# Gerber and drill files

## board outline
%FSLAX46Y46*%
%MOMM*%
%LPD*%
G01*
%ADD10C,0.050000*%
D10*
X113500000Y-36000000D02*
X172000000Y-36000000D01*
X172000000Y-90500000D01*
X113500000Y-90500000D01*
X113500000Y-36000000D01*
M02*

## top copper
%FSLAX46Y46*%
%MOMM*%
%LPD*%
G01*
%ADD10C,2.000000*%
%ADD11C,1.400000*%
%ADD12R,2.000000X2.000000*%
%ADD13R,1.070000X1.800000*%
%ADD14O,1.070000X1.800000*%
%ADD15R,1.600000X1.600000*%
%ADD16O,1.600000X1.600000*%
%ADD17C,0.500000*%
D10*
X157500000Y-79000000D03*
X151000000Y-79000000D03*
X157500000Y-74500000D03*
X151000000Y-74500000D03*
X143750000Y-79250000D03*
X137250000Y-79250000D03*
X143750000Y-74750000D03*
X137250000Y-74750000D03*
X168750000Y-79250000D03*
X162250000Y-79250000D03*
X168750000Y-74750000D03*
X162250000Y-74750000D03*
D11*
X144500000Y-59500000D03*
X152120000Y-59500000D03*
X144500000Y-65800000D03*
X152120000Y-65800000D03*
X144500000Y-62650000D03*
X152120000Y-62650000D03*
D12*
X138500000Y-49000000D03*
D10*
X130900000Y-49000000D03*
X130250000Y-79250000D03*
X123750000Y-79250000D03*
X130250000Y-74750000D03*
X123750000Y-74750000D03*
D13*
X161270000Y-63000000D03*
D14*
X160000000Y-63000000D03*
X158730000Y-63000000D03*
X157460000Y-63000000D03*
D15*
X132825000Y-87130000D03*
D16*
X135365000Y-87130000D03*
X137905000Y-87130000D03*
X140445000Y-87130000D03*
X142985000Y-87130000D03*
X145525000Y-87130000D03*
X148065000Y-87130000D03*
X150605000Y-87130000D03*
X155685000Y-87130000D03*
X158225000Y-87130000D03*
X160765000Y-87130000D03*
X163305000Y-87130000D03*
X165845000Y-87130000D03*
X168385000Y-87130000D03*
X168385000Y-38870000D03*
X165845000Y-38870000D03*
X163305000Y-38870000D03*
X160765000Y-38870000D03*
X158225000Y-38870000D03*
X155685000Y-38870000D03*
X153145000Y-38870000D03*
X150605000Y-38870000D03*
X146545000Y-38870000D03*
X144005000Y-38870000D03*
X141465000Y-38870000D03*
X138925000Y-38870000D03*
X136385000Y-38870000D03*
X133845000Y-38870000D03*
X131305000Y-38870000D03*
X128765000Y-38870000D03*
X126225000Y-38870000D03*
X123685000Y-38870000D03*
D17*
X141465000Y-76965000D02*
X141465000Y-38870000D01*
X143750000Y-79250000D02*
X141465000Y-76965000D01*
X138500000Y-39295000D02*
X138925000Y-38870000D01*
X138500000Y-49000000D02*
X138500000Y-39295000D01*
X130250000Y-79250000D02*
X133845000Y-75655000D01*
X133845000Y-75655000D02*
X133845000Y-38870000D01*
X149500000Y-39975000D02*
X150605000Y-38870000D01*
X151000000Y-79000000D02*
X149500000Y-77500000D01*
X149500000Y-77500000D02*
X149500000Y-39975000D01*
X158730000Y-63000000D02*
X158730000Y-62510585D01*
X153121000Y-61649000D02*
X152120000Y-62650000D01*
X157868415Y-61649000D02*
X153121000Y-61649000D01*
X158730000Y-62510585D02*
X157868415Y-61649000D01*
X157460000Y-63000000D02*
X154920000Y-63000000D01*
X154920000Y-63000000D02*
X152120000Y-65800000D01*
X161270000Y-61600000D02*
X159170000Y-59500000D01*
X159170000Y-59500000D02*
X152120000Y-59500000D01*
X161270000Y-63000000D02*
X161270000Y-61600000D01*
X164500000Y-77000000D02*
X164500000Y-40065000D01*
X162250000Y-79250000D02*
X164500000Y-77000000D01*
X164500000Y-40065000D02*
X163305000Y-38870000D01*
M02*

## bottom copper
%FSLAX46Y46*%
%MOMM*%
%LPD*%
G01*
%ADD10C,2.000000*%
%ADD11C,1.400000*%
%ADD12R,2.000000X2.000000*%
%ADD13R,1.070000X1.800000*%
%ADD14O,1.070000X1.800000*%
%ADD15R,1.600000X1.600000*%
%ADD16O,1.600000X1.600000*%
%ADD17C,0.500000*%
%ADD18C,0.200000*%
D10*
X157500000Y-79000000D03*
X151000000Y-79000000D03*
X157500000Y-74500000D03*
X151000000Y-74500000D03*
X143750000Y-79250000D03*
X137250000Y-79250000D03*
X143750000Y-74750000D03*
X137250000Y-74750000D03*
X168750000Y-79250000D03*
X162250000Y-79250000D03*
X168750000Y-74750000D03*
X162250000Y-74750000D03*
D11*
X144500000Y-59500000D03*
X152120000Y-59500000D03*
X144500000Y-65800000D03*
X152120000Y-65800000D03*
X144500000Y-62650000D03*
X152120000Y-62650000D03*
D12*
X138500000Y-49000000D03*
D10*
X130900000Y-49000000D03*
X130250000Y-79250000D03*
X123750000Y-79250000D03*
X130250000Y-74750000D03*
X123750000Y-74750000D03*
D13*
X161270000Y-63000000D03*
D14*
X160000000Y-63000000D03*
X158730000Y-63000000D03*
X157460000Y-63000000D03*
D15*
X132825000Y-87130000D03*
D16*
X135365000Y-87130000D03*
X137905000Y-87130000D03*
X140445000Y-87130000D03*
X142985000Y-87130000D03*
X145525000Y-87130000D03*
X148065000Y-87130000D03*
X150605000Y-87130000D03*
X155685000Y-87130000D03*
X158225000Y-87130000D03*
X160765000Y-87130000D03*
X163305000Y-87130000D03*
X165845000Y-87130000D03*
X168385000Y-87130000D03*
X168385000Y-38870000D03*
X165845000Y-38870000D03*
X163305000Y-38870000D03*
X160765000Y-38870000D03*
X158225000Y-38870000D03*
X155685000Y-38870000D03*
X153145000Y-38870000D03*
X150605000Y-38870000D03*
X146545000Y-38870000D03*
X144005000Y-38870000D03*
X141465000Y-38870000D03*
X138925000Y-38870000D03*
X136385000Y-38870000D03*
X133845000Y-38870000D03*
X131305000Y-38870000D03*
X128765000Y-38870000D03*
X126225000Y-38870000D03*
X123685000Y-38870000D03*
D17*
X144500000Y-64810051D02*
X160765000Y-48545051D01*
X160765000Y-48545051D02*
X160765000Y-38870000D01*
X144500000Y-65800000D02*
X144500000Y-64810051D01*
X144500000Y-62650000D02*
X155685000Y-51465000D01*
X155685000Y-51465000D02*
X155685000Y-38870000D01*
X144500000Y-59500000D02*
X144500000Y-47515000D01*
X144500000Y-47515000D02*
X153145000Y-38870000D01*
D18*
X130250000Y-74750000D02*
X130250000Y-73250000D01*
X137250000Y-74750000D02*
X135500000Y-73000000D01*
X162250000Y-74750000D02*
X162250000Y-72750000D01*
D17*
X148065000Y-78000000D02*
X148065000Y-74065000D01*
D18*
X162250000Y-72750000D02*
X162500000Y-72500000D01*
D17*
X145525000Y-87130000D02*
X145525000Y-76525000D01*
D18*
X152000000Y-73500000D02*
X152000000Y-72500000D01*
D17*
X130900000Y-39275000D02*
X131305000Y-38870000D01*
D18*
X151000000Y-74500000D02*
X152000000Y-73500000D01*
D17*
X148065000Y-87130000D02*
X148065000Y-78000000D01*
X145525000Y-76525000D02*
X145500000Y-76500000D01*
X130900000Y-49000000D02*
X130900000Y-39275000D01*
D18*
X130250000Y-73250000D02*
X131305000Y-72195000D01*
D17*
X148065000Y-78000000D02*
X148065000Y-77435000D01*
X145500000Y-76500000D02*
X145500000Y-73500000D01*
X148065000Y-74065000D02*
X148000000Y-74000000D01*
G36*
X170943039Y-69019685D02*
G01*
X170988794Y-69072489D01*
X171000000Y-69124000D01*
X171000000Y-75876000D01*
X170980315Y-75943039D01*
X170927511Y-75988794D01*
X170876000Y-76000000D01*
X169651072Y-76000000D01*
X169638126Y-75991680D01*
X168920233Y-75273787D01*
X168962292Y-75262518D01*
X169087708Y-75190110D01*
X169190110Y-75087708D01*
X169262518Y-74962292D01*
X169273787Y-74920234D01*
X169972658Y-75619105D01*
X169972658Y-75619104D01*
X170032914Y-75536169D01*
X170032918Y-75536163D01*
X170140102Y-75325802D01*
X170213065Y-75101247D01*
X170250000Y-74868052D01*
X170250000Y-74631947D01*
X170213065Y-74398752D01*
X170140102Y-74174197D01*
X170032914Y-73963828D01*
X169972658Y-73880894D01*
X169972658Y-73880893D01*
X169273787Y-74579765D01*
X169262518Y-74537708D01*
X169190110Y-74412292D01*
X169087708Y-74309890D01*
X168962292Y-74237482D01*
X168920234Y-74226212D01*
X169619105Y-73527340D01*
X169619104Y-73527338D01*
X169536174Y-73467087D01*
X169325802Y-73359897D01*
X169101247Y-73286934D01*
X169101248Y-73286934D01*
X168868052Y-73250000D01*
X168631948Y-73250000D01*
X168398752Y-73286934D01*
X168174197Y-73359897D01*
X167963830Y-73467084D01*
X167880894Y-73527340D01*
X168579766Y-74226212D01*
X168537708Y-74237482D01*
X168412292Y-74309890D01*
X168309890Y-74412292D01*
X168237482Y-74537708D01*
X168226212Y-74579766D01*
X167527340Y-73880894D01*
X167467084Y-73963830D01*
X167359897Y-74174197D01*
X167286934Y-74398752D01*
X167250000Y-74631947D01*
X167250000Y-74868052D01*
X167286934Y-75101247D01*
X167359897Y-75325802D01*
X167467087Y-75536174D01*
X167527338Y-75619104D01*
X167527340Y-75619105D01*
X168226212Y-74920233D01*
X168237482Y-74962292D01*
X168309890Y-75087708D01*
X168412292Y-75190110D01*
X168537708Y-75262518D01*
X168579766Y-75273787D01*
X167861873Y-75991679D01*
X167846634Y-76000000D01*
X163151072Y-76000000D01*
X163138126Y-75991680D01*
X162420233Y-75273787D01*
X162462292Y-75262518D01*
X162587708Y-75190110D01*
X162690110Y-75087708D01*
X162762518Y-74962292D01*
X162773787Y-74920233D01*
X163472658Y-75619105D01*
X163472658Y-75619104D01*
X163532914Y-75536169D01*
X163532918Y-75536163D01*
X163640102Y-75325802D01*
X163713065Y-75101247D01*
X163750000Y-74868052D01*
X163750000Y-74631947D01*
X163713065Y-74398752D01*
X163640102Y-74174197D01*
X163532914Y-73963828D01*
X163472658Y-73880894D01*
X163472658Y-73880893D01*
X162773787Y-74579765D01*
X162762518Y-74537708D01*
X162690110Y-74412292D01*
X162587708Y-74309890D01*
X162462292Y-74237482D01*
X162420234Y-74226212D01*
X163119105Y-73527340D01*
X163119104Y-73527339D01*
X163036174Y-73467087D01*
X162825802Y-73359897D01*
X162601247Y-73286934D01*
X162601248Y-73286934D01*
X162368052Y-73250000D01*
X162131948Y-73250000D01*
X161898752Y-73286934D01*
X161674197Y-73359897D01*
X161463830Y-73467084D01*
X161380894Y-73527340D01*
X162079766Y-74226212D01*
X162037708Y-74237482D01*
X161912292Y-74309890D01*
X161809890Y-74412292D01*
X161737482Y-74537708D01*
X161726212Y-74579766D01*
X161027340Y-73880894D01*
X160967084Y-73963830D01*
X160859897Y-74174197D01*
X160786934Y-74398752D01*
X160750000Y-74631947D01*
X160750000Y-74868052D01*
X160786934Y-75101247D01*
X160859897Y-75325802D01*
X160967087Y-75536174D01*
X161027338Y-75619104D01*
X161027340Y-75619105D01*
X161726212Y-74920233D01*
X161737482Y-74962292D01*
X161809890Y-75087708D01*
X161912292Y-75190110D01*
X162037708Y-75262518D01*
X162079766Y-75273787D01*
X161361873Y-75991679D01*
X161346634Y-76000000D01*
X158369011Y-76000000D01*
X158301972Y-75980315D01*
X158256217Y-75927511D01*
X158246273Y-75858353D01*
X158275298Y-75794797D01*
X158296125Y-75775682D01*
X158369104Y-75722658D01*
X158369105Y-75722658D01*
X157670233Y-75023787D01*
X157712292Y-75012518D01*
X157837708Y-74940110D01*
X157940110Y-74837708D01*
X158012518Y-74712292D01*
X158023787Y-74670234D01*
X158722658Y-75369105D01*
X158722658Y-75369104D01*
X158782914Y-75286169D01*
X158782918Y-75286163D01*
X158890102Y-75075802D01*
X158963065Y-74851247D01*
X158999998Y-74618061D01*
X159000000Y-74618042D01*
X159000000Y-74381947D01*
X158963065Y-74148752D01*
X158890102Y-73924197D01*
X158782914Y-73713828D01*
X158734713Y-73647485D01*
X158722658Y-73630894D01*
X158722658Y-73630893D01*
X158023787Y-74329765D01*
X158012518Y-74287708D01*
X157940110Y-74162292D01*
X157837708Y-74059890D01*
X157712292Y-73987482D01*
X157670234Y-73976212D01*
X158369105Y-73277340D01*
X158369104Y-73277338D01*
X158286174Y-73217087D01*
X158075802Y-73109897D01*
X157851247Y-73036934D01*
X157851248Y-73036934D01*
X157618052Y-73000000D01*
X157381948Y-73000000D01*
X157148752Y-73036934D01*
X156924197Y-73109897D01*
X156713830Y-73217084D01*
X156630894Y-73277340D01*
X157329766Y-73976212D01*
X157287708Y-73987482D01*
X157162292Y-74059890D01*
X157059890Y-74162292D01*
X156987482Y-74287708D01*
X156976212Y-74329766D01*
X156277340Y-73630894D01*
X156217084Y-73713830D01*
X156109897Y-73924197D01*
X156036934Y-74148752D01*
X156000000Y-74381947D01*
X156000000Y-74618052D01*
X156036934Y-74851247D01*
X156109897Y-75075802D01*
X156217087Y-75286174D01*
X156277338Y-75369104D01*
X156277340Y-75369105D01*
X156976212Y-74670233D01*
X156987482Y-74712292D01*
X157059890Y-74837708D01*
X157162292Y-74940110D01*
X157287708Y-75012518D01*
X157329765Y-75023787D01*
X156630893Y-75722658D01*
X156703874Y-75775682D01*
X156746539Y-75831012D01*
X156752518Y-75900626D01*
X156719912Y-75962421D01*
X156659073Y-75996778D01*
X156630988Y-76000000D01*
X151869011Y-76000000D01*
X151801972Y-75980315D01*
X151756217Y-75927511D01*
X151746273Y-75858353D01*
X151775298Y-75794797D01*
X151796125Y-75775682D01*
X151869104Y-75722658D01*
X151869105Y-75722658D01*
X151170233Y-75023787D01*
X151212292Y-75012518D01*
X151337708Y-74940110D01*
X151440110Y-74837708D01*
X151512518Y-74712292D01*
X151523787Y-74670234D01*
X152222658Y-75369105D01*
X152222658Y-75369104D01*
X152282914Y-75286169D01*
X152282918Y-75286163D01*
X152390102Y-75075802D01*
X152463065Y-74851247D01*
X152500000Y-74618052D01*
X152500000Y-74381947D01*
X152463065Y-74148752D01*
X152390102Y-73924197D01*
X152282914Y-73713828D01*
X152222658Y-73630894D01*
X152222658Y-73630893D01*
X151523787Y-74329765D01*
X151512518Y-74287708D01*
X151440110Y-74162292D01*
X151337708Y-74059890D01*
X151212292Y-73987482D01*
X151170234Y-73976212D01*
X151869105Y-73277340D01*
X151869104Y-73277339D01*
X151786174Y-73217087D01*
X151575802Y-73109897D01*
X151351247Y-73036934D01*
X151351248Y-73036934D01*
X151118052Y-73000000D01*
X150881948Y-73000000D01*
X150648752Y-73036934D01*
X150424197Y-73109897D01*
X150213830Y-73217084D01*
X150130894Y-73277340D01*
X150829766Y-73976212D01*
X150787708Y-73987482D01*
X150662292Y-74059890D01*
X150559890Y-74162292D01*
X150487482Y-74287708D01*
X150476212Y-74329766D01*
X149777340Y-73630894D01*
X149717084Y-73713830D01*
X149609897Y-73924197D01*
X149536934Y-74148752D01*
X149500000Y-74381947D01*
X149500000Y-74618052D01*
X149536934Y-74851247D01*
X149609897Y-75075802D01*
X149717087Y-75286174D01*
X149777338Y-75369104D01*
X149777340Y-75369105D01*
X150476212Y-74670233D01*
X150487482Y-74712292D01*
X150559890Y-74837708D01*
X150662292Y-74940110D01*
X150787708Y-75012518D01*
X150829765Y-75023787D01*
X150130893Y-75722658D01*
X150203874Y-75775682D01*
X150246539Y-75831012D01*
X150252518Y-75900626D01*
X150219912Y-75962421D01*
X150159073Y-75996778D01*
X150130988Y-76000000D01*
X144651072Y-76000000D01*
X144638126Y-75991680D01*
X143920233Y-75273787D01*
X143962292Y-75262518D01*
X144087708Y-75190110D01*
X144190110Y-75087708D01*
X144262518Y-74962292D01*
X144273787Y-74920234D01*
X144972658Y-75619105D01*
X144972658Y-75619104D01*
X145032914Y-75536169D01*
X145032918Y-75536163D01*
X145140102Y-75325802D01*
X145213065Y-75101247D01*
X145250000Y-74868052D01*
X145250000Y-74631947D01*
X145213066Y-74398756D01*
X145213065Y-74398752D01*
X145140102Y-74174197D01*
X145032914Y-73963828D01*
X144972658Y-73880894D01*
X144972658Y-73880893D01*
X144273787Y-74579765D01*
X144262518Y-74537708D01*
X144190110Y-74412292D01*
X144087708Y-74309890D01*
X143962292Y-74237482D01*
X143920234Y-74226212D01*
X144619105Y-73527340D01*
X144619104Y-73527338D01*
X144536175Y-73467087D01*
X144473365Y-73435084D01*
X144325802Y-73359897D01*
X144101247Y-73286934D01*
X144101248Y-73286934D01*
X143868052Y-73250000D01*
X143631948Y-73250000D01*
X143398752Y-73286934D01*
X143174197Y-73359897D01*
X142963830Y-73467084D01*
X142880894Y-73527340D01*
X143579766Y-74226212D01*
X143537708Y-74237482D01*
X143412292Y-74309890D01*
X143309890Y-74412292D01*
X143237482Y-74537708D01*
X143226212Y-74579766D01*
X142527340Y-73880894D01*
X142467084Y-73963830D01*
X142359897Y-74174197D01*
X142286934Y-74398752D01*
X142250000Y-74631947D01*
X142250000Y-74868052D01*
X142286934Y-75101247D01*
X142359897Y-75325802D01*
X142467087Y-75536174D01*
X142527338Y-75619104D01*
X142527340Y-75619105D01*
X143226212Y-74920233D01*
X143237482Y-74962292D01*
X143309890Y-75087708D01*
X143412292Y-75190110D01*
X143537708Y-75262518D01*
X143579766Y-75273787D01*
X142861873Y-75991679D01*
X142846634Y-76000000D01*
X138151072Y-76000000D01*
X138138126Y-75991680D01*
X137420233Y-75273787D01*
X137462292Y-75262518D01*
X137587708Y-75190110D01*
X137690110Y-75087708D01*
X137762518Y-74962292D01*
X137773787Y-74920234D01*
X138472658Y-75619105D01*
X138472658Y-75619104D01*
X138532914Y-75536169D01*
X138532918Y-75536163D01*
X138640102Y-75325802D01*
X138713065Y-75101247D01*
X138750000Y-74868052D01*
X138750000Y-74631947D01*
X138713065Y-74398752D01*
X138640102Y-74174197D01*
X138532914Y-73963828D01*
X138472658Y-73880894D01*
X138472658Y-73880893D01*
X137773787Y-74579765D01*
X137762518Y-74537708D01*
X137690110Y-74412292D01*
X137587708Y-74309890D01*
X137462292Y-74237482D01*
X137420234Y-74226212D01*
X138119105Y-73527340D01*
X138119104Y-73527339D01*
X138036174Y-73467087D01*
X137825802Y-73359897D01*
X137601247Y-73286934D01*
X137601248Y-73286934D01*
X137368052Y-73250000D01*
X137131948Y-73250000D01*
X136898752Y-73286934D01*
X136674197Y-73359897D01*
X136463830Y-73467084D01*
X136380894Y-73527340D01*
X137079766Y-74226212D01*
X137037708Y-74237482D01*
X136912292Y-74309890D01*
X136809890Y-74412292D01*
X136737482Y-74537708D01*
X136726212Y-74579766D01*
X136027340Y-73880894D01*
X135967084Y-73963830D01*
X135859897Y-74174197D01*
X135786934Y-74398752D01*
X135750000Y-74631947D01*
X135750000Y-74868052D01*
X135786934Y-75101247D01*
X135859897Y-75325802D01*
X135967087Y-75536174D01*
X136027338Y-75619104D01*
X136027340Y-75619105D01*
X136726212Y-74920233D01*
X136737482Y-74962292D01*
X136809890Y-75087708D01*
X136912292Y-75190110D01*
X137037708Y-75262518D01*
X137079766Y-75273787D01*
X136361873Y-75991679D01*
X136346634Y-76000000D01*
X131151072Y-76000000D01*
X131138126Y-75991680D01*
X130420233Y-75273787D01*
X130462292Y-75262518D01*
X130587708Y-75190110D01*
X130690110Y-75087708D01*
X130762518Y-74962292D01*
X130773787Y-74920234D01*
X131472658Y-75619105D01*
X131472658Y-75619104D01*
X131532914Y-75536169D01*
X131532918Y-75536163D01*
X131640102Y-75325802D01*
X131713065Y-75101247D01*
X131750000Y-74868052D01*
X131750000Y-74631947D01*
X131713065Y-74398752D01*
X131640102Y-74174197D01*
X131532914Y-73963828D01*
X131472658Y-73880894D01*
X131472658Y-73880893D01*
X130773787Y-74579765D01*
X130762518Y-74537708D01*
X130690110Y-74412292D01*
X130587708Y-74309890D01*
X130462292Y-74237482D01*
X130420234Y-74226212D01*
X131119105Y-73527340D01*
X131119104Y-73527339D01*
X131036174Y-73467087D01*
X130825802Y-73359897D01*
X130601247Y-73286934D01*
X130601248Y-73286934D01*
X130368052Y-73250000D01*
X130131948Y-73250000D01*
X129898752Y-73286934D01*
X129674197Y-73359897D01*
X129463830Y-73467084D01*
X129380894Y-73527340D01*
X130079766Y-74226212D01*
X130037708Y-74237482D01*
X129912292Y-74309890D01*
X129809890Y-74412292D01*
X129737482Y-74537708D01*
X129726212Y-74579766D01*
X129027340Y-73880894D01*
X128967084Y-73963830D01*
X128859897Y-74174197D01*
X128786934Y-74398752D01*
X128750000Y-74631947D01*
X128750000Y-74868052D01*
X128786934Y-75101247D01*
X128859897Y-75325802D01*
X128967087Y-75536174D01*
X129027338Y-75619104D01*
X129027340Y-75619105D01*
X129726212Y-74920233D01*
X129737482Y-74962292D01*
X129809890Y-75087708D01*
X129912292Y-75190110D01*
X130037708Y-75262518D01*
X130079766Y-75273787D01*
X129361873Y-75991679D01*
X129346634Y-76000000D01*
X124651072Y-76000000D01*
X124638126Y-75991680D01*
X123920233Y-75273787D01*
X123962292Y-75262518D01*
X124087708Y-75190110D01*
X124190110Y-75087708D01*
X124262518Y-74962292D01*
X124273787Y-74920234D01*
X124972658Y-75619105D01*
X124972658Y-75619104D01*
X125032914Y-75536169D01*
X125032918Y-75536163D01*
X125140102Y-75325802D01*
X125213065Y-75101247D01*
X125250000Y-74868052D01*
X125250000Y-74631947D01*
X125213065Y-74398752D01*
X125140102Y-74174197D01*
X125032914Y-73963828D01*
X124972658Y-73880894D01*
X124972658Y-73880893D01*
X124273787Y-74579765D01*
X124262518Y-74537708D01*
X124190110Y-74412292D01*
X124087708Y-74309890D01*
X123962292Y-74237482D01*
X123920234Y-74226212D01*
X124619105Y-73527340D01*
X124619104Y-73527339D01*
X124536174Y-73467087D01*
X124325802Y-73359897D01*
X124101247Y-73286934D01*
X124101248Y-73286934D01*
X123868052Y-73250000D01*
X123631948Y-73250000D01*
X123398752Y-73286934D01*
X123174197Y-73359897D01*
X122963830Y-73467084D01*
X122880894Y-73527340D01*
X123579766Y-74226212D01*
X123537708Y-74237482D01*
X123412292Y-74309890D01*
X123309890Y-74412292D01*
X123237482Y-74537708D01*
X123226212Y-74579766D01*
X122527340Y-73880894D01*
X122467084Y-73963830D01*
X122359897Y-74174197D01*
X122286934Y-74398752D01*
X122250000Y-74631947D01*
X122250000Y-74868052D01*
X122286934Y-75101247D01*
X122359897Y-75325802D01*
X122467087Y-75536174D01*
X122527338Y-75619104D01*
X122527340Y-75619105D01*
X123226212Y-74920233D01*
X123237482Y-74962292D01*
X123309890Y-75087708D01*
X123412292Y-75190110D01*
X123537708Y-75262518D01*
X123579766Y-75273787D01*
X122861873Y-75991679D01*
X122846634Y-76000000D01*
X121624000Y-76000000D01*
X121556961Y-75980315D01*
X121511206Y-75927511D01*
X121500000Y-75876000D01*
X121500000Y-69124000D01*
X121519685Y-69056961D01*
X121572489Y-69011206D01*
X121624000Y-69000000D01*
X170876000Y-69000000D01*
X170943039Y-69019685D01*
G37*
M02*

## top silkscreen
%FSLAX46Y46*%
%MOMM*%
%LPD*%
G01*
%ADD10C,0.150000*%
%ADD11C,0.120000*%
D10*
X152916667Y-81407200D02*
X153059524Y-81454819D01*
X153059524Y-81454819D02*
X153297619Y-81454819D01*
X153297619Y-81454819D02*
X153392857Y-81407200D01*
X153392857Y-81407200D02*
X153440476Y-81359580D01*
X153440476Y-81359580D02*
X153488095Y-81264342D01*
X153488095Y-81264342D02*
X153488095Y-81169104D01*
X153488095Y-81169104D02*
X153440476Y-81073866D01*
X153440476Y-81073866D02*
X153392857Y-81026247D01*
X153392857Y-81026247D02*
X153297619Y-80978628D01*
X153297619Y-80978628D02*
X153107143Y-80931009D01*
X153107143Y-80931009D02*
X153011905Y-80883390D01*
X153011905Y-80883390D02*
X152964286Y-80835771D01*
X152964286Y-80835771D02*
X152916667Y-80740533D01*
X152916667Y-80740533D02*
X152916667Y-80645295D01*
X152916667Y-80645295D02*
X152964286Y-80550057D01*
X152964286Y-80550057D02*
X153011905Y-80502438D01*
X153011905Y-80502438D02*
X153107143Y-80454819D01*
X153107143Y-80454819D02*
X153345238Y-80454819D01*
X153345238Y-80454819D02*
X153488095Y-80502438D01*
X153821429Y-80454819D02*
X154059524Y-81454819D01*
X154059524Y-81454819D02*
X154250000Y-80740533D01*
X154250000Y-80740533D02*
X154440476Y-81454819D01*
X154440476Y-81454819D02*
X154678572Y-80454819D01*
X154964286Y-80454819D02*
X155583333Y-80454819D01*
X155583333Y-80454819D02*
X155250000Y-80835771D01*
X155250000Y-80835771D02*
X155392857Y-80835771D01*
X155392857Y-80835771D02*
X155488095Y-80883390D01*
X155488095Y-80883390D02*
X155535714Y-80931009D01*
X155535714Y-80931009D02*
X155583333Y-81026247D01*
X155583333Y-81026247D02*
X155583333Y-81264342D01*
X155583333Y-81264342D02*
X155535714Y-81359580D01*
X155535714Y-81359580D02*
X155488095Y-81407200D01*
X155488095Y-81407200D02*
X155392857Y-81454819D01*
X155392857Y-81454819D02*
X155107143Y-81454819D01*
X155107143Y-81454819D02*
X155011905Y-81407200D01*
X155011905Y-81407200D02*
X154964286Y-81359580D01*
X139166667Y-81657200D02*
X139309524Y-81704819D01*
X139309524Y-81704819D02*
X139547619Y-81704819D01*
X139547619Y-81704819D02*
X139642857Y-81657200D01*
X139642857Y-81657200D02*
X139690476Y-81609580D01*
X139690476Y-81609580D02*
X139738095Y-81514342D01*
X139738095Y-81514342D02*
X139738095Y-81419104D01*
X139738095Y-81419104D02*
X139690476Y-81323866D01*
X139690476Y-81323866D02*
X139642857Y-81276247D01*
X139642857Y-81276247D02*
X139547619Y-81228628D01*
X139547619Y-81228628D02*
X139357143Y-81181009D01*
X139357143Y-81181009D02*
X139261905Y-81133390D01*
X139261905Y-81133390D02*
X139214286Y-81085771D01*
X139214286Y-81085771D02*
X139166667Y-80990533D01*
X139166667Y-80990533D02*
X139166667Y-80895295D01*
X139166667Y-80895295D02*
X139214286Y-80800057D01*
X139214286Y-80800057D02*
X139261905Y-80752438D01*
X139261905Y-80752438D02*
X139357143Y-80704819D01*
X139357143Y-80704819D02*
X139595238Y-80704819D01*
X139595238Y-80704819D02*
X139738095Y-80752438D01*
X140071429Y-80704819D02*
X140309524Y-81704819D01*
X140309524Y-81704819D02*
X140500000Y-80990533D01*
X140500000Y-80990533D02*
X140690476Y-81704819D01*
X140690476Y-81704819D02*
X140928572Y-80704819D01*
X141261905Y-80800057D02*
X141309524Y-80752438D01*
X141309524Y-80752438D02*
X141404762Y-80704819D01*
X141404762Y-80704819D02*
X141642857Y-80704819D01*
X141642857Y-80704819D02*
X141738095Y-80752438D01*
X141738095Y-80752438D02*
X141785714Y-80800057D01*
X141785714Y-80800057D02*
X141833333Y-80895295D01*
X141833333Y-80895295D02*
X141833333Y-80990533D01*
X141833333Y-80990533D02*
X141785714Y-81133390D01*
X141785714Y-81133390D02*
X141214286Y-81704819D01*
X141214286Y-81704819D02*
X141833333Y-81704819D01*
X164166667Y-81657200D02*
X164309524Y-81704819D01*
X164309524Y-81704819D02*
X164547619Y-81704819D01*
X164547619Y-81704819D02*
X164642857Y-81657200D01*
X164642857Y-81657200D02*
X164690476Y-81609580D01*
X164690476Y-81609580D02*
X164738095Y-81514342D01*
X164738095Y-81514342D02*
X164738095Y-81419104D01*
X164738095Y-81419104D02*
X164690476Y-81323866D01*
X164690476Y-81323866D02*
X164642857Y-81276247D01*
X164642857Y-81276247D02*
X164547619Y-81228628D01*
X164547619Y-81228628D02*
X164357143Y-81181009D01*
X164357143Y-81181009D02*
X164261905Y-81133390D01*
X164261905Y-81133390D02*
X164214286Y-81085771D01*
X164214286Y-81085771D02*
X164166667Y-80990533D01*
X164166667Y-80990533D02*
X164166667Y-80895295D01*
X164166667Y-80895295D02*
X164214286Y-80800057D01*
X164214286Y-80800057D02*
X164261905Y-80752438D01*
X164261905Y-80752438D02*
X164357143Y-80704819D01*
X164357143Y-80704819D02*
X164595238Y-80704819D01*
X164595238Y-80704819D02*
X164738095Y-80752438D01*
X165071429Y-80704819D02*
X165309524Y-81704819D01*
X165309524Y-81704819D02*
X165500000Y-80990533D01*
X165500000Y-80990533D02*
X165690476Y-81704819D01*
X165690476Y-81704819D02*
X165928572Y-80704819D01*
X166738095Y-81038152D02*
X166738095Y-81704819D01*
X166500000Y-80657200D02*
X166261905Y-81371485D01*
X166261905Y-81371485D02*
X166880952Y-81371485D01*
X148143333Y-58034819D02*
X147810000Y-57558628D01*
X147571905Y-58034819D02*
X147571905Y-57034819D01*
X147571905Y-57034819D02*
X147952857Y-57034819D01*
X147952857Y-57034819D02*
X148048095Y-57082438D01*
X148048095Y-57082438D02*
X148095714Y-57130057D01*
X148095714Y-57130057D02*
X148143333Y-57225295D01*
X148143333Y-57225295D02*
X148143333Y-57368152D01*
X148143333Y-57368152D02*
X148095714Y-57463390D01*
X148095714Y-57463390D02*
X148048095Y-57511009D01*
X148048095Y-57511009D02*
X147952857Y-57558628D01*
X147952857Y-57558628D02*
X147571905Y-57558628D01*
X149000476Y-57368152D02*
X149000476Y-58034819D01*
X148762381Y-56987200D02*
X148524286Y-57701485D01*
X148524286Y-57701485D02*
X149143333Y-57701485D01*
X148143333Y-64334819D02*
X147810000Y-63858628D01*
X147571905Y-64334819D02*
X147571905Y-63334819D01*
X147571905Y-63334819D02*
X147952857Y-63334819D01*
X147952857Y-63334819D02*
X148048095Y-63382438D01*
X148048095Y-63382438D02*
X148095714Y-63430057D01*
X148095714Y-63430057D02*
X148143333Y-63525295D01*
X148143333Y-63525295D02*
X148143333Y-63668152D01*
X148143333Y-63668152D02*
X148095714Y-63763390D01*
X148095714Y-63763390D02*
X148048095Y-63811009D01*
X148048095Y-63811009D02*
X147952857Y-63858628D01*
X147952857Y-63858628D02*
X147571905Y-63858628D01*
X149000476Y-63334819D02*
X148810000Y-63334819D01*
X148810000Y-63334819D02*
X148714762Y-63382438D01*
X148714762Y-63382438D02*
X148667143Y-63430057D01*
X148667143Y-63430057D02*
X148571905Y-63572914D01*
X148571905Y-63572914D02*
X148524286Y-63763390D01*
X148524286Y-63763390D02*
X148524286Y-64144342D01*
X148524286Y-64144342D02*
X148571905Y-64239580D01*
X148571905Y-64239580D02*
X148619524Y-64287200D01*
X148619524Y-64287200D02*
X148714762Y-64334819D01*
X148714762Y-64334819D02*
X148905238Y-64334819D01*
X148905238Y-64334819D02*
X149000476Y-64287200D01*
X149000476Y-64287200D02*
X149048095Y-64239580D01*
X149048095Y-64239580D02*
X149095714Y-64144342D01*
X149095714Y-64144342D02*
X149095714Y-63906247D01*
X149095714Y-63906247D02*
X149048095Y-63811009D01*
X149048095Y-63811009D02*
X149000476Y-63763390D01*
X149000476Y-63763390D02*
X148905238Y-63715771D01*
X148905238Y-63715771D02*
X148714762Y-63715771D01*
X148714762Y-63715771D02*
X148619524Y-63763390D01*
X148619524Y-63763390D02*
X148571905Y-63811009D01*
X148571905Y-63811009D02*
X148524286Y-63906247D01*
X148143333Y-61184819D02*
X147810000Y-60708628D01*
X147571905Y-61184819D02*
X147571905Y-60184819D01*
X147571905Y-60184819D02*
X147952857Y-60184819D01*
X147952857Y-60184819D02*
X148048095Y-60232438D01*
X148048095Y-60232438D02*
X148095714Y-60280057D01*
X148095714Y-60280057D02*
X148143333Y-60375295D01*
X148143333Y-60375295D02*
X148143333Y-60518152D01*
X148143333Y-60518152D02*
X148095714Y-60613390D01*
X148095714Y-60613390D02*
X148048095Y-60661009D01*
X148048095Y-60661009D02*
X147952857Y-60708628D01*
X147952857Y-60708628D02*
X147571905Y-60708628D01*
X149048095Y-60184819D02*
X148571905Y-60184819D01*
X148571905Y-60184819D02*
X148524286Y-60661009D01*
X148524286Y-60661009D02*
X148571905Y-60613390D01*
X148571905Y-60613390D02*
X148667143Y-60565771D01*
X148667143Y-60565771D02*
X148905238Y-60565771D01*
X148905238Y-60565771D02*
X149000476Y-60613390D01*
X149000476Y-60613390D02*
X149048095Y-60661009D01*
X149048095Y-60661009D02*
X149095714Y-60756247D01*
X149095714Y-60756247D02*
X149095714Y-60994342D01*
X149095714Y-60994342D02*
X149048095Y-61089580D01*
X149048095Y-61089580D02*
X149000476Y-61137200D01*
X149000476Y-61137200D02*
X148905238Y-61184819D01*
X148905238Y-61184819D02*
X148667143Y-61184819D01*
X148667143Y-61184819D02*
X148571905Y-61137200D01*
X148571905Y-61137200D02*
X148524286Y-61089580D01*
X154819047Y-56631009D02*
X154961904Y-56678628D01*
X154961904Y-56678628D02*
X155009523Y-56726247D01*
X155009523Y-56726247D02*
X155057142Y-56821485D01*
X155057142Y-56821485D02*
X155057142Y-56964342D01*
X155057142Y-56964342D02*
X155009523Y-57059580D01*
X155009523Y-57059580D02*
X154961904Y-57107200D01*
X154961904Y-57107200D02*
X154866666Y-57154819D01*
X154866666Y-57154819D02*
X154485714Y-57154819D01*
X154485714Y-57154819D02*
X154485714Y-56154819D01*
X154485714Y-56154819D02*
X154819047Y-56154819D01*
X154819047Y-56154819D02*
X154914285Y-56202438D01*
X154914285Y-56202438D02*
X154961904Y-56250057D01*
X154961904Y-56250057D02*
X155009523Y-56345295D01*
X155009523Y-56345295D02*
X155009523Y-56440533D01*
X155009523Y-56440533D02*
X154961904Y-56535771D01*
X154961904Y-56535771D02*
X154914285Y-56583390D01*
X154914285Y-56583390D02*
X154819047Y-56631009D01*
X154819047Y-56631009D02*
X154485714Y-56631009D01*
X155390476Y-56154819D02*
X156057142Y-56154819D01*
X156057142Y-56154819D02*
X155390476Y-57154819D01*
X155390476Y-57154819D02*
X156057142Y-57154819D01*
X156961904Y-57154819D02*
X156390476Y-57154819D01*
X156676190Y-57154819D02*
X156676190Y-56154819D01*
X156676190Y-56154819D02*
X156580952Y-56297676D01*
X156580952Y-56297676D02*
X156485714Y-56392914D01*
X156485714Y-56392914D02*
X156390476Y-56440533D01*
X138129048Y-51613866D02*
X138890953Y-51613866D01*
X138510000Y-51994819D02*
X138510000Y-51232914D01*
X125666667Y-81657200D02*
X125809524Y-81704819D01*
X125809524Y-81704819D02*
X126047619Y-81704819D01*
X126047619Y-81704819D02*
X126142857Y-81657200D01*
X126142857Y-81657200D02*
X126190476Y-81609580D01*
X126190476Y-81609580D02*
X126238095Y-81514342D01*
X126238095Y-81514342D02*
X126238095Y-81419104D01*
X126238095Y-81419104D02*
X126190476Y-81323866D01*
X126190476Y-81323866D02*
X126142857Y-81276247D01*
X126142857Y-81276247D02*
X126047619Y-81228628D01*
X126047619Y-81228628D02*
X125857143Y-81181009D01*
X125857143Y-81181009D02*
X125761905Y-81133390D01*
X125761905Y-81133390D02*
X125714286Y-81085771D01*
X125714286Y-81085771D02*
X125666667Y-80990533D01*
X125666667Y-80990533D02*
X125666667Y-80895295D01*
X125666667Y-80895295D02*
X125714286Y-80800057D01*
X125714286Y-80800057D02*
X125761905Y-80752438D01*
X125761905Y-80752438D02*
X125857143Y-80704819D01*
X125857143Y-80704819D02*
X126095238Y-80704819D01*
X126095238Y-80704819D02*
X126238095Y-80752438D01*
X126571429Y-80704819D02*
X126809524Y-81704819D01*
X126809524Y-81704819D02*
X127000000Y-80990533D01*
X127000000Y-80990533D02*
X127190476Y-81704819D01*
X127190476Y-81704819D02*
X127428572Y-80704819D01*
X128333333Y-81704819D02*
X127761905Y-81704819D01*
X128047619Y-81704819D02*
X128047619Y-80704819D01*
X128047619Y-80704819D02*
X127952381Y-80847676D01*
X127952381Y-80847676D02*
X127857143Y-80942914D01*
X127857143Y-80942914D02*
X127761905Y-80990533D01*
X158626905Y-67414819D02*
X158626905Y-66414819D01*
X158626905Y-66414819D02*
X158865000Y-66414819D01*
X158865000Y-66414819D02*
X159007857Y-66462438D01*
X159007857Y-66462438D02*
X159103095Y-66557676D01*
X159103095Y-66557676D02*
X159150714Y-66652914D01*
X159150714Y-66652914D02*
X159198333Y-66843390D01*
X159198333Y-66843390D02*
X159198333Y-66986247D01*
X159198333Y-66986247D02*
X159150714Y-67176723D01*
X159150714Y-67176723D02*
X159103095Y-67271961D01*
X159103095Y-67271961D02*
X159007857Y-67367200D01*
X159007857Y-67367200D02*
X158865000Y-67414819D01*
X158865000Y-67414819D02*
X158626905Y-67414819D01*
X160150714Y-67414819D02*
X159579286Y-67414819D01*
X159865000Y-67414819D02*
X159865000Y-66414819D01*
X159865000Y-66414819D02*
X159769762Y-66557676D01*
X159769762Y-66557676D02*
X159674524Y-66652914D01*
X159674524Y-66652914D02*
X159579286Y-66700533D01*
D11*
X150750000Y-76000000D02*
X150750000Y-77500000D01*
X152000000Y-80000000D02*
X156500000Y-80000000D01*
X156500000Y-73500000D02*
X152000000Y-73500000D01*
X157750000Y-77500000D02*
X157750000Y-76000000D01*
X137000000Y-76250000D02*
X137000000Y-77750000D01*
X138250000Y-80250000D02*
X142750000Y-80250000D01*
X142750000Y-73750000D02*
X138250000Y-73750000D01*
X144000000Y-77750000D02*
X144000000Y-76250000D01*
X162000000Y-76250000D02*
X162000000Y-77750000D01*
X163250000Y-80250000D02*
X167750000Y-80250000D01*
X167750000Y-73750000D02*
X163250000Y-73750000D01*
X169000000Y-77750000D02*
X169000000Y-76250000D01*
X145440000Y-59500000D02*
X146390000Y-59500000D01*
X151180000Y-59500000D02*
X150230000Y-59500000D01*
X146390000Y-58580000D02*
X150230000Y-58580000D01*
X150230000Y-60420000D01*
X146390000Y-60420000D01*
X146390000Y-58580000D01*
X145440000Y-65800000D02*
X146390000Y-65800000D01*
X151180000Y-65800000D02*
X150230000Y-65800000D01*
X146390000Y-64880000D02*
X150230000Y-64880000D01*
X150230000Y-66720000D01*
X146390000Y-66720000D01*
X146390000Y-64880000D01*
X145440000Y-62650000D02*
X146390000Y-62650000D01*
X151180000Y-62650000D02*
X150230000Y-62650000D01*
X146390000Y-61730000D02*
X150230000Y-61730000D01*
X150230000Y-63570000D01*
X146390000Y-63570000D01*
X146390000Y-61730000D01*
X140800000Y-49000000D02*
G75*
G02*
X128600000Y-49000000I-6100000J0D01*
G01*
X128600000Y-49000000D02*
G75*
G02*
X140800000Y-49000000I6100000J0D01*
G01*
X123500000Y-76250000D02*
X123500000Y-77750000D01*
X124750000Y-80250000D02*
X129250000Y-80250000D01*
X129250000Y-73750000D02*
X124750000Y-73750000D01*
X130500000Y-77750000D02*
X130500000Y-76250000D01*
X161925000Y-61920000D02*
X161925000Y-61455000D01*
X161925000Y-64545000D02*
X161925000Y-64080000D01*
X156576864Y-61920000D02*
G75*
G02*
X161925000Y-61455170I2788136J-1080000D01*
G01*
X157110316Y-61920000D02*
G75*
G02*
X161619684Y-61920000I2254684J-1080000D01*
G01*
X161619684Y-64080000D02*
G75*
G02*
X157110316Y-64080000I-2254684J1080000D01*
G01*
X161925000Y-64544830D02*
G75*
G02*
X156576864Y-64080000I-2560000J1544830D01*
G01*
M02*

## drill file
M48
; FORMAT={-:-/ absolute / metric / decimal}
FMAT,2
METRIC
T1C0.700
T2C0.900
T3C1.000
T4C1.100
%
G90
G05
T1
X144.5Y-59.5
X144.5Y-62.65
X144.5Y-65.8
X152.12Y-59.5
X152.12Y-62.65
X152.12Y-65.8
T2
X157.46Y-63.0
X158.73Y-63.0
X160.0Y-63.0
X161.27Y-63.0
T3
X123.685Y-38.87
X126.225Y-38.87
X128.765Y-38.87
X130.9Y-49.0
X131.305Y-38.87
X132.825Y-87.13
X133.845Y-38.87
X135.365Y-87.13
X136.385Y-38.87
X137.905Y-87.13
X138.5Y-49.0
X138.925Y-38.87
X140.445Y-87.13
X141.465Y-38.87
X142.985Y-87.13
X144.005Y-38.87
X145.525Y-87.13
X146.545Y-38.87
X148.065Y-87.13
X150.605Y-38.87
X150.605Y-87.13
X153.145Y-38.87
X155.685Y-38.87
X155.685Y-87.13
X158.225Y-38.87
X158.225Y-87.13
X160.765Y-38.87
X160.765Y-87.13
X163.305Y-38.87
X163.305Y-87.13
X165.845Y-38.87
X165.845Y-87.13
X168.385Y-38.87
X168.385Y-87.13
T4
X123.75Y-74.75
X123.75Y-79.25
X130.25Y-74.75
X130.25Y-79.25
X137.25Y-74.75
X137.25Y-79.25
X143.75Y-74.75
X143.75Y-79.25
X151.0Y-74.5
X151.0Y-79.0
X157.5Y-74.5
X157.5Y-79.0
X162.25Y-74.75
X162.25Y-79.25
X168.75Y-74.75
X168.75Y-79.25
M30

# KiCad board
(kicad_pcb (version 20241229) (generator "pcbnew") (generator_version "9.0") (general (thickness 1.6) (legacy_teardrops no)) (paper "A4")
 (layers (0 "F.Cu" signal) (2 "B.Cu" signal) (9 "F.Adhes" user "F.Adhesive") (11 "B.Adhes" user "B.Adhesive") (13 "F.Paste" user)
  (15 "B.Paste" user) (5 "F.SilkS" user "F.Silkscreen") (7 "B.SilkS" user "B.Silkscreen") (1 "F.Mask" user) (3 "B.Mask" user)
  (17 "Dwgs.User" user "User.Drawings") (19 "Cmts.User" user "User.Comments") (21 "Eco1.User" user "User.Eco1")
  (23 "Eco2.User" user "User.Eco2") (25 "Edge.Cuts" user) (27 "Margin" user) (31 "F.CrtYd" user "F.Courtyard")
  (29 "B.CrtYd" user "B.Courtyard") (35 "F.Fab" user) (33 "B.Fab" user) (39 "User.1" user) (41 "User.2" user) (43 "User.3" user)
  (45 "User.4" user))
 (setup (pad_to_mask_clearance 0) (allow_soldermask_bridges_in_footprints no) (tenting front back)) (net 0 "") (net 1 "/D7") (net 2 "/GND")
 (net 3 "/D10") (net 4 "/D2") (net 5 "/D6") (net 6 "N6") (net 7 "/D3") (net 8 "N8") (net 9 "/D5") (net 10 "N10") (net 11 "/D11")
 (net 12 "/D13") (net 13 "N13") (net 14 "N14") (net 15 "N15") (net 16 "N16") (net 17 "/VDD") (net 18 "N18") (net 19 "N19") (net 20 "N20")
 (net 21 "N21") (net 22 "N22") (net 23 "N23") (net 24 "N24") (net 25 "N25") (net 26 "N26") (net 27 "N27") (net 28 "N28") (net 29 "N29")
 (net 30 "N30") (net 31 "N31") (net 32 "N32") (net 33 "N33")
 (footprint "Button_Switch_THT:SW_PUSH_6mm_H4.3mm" (layer "F.Cu") (at 157.5 79 180)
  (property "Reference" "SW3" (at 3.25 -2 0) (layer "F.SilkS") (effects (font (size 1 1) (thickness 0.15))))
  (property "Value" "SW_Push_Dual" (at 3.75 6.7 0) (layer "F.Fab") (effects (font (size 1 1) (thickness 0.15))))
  (fp_line (start 6.75 3) (end 6.75 1.5) (stroke (width 0.12) (type solid)) (layer "F.SilkS"))
  (fp_line (start 5.5 -1) (end 1 -1) (stroke (width 0.12) (type solid)) (layer "F.SilkS"))
  (fp_line (start 1 5.5) (end 5.5 5.5) (stroke (width 0.12) (type solid)) (layer "F.SilkS"))
  (fp_line (start -0.25 1.5) (end -0.25 3) (stroke (width 0.12) (type solid)) (layer "F.SilkS"))
  (pad "1" thru_hole circle (at 0 0 270) (size 2 2) (drill 1.1) (layers "*.Cu" "*.Mask") (remove_unused_layers no) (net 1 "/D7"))
  (pad "1" thru_hole circle (at 6.5 0 270) (size 2 2) (drill 1.1) (layers "*.Cu" "*.Mask") (remove_unused_layers no) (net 1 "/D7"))
  (pad "2" thru_hole circle (at 0 4.5 270) (size 2 2) (drill 1.1) (layers "*.Cu" "*.Mask") (remove_unused_layers no) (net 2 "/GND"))
  (pad "2" thru_hole circle (at 6.5 4.5 270) (size 2 2) (drill 1.1) (layers "*.Cu" "*.Mask") (remove_unused_layers no) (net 2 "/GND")))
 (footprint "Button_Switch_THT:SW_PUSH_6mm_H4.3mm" (layer "F.Cu") (at 143.75 79.25 180)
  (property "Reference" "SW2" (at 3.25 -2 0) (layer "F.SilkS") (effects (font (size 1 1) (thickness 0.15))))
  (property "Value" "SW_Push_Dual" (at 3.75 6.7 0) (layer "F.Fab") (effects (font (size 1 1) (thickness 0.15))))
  (fp_line (start 6.75 3) (end 6.75 1.5) (stroke (width 0.12) (type solid)) (layer "F.SilkS"))
  (fp_line (start 5.5 -1) (end 1 -1) (stroke (width 0.12) (type solid)) (layer "F.SilkS"))
  (fp_line (start 1 5.5) (end 5.5 5.5) (stroke (width 0.12) (type solid)) (layer "F.SilkS"))
  (fp_line (start -0.25 1.5) (end -0.25 3) (stroke (width 0.12) (type solid)) (layer "F.SilkS"))
  (pad "1" thru_hole circle (at 0 0 270) (size 2 2) (drill 1.1) (layers "*.Cu" "*.Mask") (remove_unused_layers no) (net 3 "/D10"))
  (pad "1" thru_hole circle (at 6.5 0 270) (size 2 2) (drill 1.1) (layers "*.Cu" "*.Mask") (remove_unused_layers no) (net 3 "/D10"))
  (pad "2" thru_hole circle (at 0 4.5 270) (size 2 2) (drill 1.1) (layers "*.Cu" "*.Mask") (remove_unused_layers no) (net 2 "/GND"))
  (pad "2" thru_hole circle (at 6.5 4.5 270) (size 2 2) (drill 1.1) (layers "*.Cu" "*.Mask") (remove_unused_layers no) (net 2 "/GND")))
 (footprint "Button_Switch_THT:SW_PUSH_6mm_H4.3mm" (layer "F.Cu") (at 168.75 79.25 180)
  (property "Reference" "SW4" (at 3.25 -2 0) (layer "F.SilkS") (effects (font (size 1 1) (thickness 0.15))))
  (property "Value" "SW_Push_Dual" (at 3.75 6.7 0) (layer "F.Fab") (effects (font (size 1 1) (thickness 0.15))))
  (fp_line (start 6.75 3) (end 6.75 1.5) (stroke (width 0.12) (type solid)) (layer "F.SilkS"))
  (fp_line (start 5.5 -1) (end 1 -1) (stroke (width 0.12) (type solid)) (layer "F.SilkS"))
  (fp_line (start 1 5.5) (end 5.5 5.5) (stroke (width 0.12) (type solid)) (layer "F.SilkS"))
  (fp_line (start -0.25 1.5) (end -0.25 3) (stroke (width 0.12) (type solid)) (layer "F.SilkS"))
  (pad "1" thru_hole circle (at 0 0 270) (size 2 2) (drill 1.1) (layers "*.Cu" "*.Mask") (remove_unused_layers no) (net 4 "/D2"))
  (pad "1" thru_hole circle (at 6.5 0 270) (size 2 2) (drill 1.1) (layers "*.Cu" "*.Mask") (remove_unused_layers no) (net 4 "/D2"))
  (pad "2" thru_hole circle (at 0 4.5 270) (size 2 2) (drill 1.1) (layers "*.Cu" "*.Mask") (remove_unused_layers no) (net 2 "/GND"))
  (pad "2" thru_hole circle (at 6.5 4.5 270) (size 2 2) (drill 1.1) (layers "*.Cu" "*.Mask") (remove_unused_layers no) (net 2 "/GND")))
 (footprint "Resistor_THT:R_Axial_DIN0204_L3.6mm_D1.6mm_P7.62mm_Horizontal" (layer "F.Cu") (at 144.5 59.5)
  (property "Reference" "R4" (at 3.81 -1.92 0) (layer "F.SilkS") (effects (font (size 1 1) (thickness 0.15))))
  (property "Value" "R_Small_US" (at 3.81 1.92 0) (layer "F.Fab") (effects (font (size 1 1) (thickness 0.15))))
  (fp_line (start 0.94 0) (end 1.89 0) (stroke (width 0.12) (type solid)) (layer "F.SilkS"))
  (fp_line (start 6.68 0) (end 5.73 0) (stroke (width 0.12) (type solid)) (layer "F.SilkS"))
  (fp_rect (start 1.89 -0.92) (end 5.73 0.92) (stroke (width 0.12) (type solid)) (fill no) (layer "F.SilkS"))
  (pad "1" thru_hole circle (at 0 0) (size 1.4 1.4) (drill 0.7) (layers "*.Cu" "*.Mask") (remove_unused_layers no) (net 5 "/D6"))
  (pad "2" thru_hole circle (at 7.62 0) (size 1.4 1.4) (drill 0.7) (layers "*.Cu" "*.Mask") (remove_unused_layers no) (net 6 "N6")))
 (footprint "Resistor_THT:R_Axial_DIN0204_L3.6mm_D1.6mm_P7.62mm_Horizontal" (layer "F.Cu") (at 144.5 65.8)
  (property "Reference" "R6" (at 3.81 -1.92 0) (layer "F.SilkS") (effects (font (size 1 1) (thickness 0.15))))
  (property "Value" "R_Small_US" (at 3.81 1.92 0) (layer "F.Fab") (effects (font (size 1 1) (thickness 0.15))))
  (fp_line (start 0.94 0) (end 1.89 0) (stroke (width 0.12) (type solid)) (layer "F.SilkS"))
  (fp_line (start 6.68 0) (end 5.73 0) (stroke (width 0.12) (type solid)) (layer "F.SilkS"))
  (fp_rect (start 1.89 -0.92) (end 5.73 0.92) (stroke (width 0.12) (type solid)) (fill no) (layer "F.SilkS"))
  (pad "1" thru_hole circle (at 0 0) (size 1.4 1.4) (drill 0.7) (layers "*.Cu" "*.Mask") (remove_unused_layers no) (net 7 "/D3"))
  (pad "2" thru_hole circle (at 7.62 0) (size 1.4 1.4) (drill 0.7) (layers "*.Cu" "*.Mask") (remove_unused_layers no) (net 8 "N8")))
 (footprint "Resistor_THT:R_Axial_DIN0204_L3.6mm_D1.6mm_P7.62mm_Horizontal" (layer "F.Cu") (at 144.5 62.65)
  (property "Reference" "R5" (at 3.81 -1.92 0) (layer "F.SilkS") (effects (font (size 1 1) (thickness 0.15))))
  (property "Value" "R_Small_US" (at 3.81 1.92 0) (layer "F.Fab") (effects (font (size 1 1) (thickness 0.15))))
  (fp_line (start 0.94 0) (end 1.89 0) (stroke (width 0.12) (type solid)) (layer "F.SilkS"))
  (fp_line (start 6.68 0) (end 5.73 0) (stroke (width 0.12) (type solid)) (layer "F.SilkS"))
  (fp_rect (start 1.89 -0.92) (end 5.73 0.92) (stroke (width 0.12) (type solid)) (fill no) (layer "F.SilkS"))
  (pad "1" thru_hole circle (at 0 0) (size 1.4 1.4) (drill 0.7) (layers "*.Cu" "*.Mask") (remove_unused_layers no) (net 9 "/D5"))
  (pad "2" thru_hole circle (at 7.62 0) (size 1.4 1.4) (drill 0.7) (layers "*.Cu" "*.Mask") (remove_unused_layers no) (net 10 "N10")))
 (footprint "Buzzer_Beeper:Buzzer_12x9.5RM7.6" (layer "F.Cu") (at 138.5 49 180)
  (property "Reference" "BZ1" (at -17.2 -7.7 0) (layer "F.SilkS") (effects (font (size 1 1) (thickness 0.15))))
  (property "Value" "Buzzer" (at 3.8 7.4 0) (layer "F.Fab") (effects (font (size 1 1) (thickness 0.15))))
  (fp_circle (center 3.8 0) (end 9.9 0) (stroke (width 0.12) (type solid)) (fill no) (layer "F.SilkS"))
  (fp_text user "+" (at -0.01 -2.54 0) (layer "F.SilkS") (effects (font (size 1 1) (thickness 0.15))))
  (pad "1" thru_hole rect (at 0 0 180) (size 2 2) (drill 1) (layers "*.Cu" "*.Mask") (remove_unused_layers no) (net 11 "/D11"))
  (pad "2" thru_hole circle (at 7.6 0 180) (size 2 2) (drill 1) (layers "*.Cu" "*.Mask") (remove_unused_layers no) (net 2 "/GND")))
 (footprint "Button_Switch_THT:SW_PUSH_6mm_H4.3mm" (layer "F.Cu") (at 130.25 79.25 180)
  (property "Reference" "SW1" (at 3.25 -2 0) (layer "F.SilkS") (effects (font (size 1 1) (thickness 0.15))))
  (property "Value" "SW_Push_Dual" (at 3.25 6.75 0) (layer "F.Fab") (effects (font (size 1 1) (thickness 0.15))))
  (fp_line (start 6.75 3) (end 6.75 1.5) (stroke (width 0.12) (type solid)) (layer "F.SilkS"))
  (fp_line (start 5.5 -1) (end 1 -1) (stroke (width 0.12) (type solid)) (layer "F.SilkS"))
  (fp_line (start 1 5.5) (end 5.5 5.5) (stroke (width 0.12) (type solid)) (layer "F.SilkS"))
  (fp_line (start -0.25 1.5) (end -0.25 3) (stroke (width 0.12) (type solid)) (layer "F.SilkS"))
  (pad "1" thru_hole circle (at 0 0 270) (size 2 2) (drill 1.1) (layers "*.Cu" "*.Mask") (remove_unused_layers no) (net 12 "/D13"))
  (pad "1" thru_hole circle (at 6.5 0 270) (size 2 2) (drill 1.1) (layers "*.Cu" "*.Mask") (remove_unused_layers no) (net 12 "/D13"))
  (pad "2" thru_hole circle (at 0 4.5 270) (size 2 2) (drill 1.1) (layers "*.Cu" "*.Mask") (remove_unused_layers no) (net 2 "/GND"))
  (pad "2" thru_hole circle (at 6.5 4.5 270) (size 2 2) (drill 1.1) (layers "*.Cu" "*.Mask") (remove_unused_layers no) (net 2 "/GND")))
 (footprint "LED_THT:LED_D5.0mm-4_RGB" (layer "F.Cu") (at 161.27 63 180)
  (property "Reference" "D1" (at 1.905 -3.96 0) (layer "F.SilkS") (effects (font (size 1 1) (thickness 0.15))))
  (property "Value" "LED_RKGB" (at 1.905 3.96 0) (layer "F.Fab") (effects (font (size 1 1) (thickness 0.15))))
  (fp_line (start -0.655 1.08) (end -0.655 1.545) (stroke (width 0.12) (type solid)) (layer "F.SilkS"))
  (fp_line (start -0.655 -1.545) (end -0.655 -1.08) (stroke (width 0.12) (type solid)) (layer "F.SilkS"))
  (fp_arc (start 4.693136 1.08) (mid 2.163898 2.97877) (end -0.655 1.54483) (stroke (width 0.12) (type solid)) (layer "F.SilkS"))
  (fp_arc (start 4.159684 1.08) (mid 1.905 2.5) (end -0.349684 1.08) (stroke (width 0.12) (type solid)) (layer "F.SilkS"))
  (fp_arc (start -0.349684 -1.08) (mid 1.905 -2.5) (end 4.159684 -1.08) (stroke (width 0.12) (type solid)) (layer "F.SilkS"))
  (fp_arc (start -0.655 -1.54483) (mid 2.163898 -2.97877) (end 4.693136 -1.08) (stroke (width 0.12) (type solid)) (layer "F.SilkS"))
  (pad "1" thru_hole rect (at 0 0 180) (size 1.07 1.8) (drill 0.9) (layers "*.Cu" "*.Mask") (remove_unused_layers no) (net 6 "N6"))
  (pad "2" thru_hole oval (at 1.27 0 180) (size 1.07 1.8) (drill 0.9) (layers "*.Cu" "*.Mask") (remove_unused_layers no) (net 2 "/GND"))
  (pad "3" thru_hole oval (at 2.54 0 180) (size 1.07 1.8) (drill 0.9) (layers "*.Cu" "*.Mask") (remove_unused_layers no) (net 10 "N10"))
  (pad "4" thru_hole oval (at 3.81 0 180) (size 1.07 1.8) (drill 0.9) (layers "*.Cu" "*.Mask") (remove_unused_layers no) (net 8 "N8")))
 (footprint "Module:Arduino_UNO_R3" (layer "B.Cu") (at 132.825 87.13)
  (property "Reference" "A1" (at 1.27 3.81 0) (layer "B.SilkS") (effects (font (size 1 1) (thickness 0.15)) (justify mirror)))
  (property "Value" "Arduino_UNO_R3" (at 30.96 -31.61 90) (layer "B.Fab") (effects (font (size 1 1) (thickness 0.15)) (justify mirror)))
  (pad "1" thru_hole rect (at 0 0 270) (size 1.6 1.6) (drill 1) (layers "*.Cu" "*.Mask") (remove_unused_layers no) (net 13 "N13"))
  (pad "2" thru_hole oval (at 2.54 0 270) (size 1.6 1.6) (drill 1) (layers "*.Cu" "*.Mask") (remove_unused_layers no) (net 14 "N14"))
  (pad "3" thru_hole oval (at 5.08 0 270) (size 1.6 1.6) (drill 1) (layers "*.Cu" "*.Mask") (remove_unused_layers no) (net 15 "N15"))
  (pad "4" thru_hole oval (at 7.62 0 270) (size 1.6 1.6) (drill 1) (layers "*.Cu" "*.Mask") (remove_unused_layers no) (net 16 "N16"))
  (pad "5" thru_hole oval (at 10.16 0 270) (size 1.6 1.6) (drill 1) (layers "*.Cu" "*.Mask") (remove_unused_layers no) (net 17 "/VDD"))
  (pad "6" thru_hole oval (at 12.7 0 270) (size 1.6 1.6) (drill 1) (layers "*.Cu" "*.Mask") (remove_unused_layers no) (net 2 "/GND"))
  (pad "7" thru_hole oval (at 15.24 0 270) (size 1.6 1.6) (drill 1) (layers "*.Cu" "*.Mask") (remove_unused_layers no) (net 2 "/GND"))
  (pad "8" thru_hole oval (at 17.78 0 270) (size 1.6 1.6) (drill 1) (layers "*.Cu" "*.Mask") (remove_unused_layers no) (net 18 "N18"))
  (pad "9" thru_hole oval (at 22.86 0 270) (size 1.6 1.6) (drill 1) (layers "*.Cu" "*.Mask") (remove_unused_layers no) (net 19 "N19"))
  (pad "10" thru_hole oval (at 25.4 0 270) (size 1.6 1.6) (drill 1) (layers "*.Cu" "*.Mask") (remove_unused_layers no) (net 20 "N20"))
  (pad "11" thru_hole oval (at 27.94 0 270) (size 1.6 1.6) (drill 1) (layers "*.Cu" "*.Mask") (remove_unused_layers no) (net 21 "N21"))
  (pad "12" thru_hole oval (at 30.48 0 270) (size 1.6 1.6) (drill 1) (layers "*.Cu" "*.Mask") (remove_unused_layers no) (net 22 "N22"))
  (pad "13" thru_hole oval (at 33.02 0 270) (size 1.6 1.6) (drill 1) (layers "*.Cu" "*.Mask") (remove_unused_layers no) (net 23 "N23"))
  (pad "14" thru_hole oval (at 35.56 0 270) (size 1.6 1.6) (drill 1) (layers "*.Cu" "*.Mask") (remove_unused_layers no) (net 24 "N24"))
  (pad "15" thru_hole oval (at 35.56 -48.26 270) (size 1.6 1.6) (drill 1) (layers "*.Cu" "*.Mask") (remove_unused_layers no) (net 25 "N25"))
  (pad "16" thru_hole oval (at 33.02 -48.26 270) (size 1.6 1.6) (drill 1) (layers "*.Cu" "*.Mask") (remove_unused_layers no) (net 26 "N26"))
  (pad "17" thru_hole oval (at 30.48 -48.26 270) (size 1.6 1.6) (drill 1) (layers "*.Cu" "*.Mask") (remove_unused_layers no) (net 4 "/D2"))
  (pad "18" thru_hole oval (at 27.94 -48.26 270) (size 1.6 1.6) (drill 1) (layers "*.Cu" "*.Mask") (remove_unused_layers no) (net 7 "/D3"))
  (pad "19" thru_hole oval (at 25.4 -48.26 270) (size 1.6 1.6) (drill 1) (layers "*.Cu" "*.Mask") (remove_unused_layers no) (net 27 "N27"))
  (pad "20" thru_hole oval (at 22.86 -48.26 270) (size 1.6 1.6) (drill 1) (layers "*.Cu" "*.Mask") (remove_unused_layers no) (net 9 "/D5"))
  (pad "21" thru_hole oval (at 20.32 -48.26 270) (size 1.6 1.6) (drill 1) (layers "*.Cu" "*.Mask") (remove_unused_layers no) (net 5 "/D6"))
  (pad "22" thru_hole oval (at 17.78 -48.26 270) (size 1.6 1.6) (drill 1) (layers "*.Cu" "*.Mask") (remove_unused_layers no) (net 20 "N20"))
  (pad "23" thru_hole oval (at 13.72 -48.26 270) (size 1.6 1.6) (drill 1) (layers "*.Cu" "*.Mask") (remove_unused_layers no) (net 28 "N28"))
  (pad "24" thru_hole oval (at 11.18 -48.26 270) (size 1.6 1.6) (drill 1) (layers "*.Cu" "*.Mask") (remove_unused_layers no) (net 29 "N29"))
  (pad "25" thru_hole oval (at 8.64 -48.26 270) (size 1.6 1.6) (drill 1) (layers "*.Cu" "*.Mask") (remove_unused_layers no) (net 3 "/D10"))
  (pad "26" thru_hole oval (at 6.1 -48.26 270) (size 1.6 1.6) (drill 1) (layers "*.Cu" "*.Mask") (remove_unused_layers no) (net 11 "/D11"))
  (pad "27" thru_hole oval (at 3.56 -48.26 270) (size 1.6 1.6) (drill 1) (layers "*.Cu" "*.Mask") (remove_unused_layers no) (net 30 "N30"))
  (pad "28" thru_hole oval (at 1.02 -48.26 270) (size 1.6 1.6) (drill 1) (layers "*.Cu" "*.Mask") (remove_unused_layers no) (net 12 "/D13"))
  (pad "29" thru_hole oval (at -1.52 -48.26 270) (size 1.6 1.6) (drill 1) (layers "*.Cu" "*.Mask") (remove_unused_layers no) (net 2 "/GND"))
  (pad "30" thru_hole oval (at -4.06 -48.26 270) (size 1.6 1.6) (drill 1) (layers "*.Cu" "*.Mask") (remove_unused_layers no) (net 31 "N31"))
  (pad "31" thru_hole oval (at -6.6 -48.26 270) (size 1.6 1.6) (drill 1) (layers "*.Cu" "*.Mask") (remove_unused_layers no) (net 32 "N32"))
  (pad "32" thru_hole oval (at -9.14 -48.26 270) (size 1.6 1.6) (drill 1) (layers "*.Cu" "*.Mask") (remove_unused_layers no) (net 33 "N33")))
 (gr_rect (start 113.5 36) (end 172 90.5) (stroke (width 0.05) (type default)) (fill no) (layer "Edge.Cuts"))
 (segment (start 144.5 64.810051) (end 160.765 48.545051) (width 0.5) (layer "B.Cu") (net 7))
 (segment (start 160.765 48.545051) (end 160.765 38.87) (width 0.5) (layer "B.Cu") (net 7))
 (segment (start 144.5 65.8) (end 144.5 64.810051) (width 0.5) (layer "B.Cu") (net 7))
 (segment (start 141.465 76.965) (end 141.465 38.87) (width 0.5) (layer "F.Cu") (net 3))
 (segment (start 143.75 79.25) (end 141.465 76.965) (width 0.5) (layer "F.Cu") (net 3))
 (segment (start 144.5 62.65) (end 155.685 51.465) (width 0.5) (layer "B.Cu") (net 9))
 (segment (start 155.685 51.465) (end 155.685 38.87) (width 0.5) (layer "B.Cu") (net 9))
 (segment (start 144.5 59.5) (end 144.5 47.515) (width 0.5) (layer "B.Cu") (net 5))
 (segment (start 144.5 47.515) (end 153.145 38.87) (width 0.5) (layer "B.Cu") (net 5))
 (segment (start 138.5 39.295) (end 138.925 38.87) (width 0.5) (layer "F.Cu") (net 11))
 (segment (start 138.5 49) (end 138.5 39.295) (width 0.5) (layer "F.Cu") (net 11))
 (segment (start 130.25 79.25) (end 133.845 75.655) (width 0.5) (layer "F.Cu") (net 12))
 (segment (start 133.845 75.655) (end 133.845 38.87) (width 0.5) (layer "F.Cu") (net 12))
 (segment (start 130.25 74.75) (end 130.25 73.25) (width 0.2) (layer "B.Cu") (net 2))
 (segment (start 137.25 74.75) (end 135.5 73) (width 0.2) (layer "B.Cu") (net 2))
 (segment (start 162.25 74.75) (end 162.25 72.75) (width 0.2) (layer "B.Cu") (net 2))
 (segment (start 148.065 78) (end 148.065 74.065) (width 0.5) (layer "B.Cu") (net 2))
 (segment (start 162.25 72.75) (end 162.5 72.5) (width 0.2) (layer "B.Cu") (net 2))
 (segment (start 145.525 87.13) (end 145.525 76.525) (width 0.5) (layer "B.Cu") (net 2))
 (segment (start 152 73.5) (end 152 72.5) (width 0.2) (layer "B.Cu") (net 2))
 (segment (start 130.9 39.275) (end 131.305 38.87) (width 0.5) (layer "B.Cu") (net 2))
 (segment (start 151 74.5) (end 152 73.5) (width 0.2) (layer "B.Cu") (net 2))
 (segment (start 148.065 87.13) (end 148.065 78) (width 0.5) (layer "B.Cu") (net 2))
 (segment (start 145.525 76.525) (end 145.5 76.5) (width 0.5) (layer "B.Cu") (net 2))
 (segment (start 130.9 49) (end 130.9 39.275) (width 0.5) (layer "B.Cu") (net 2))
 (segment (start 130.25 73.25) (end 131.305 72.195) (width 0.2) (layer "B.Cu") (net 2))
 (segment (start 148.065 78) (end 148.065 77.435) (width 0.5) (layer "B.Cu") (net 2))
 (segment (start 145.5 76.5) (end 145.5 73.5) (width 0.5) (layer "B.Cu") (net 2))
 (segment (start 148.065 74.065) (end 148 74) (width 0.5) (layer "B.Cu") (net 2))
 (segment (start 149.5 39.975) (end 150.605 38.87) (width 0.5) (layer "F.Cu") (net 1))
 (segment (start 151 79) (end 149.5 77.5) (width 0.5) (layer "F.Cu") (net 1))
 (segment (start 149.5 77.5) (end 149.5 39.975) (width 0.5) (layer "F.Cu") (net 1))
 (segment (start 158.73 63) (end 158.73 62.510585) (width 0.5) (layer "F.Cu") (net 10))
 (segment (start 153.121 61.649) (end 152.12 62.65) (width 0.5) (layer "F.Cu") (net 10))
 (segment (start 157.868415 61.649) (end 153.121 61.649) (width 0.5) (layer "F.Cu") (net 10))
 (segment (start 158.73 62.510585) (end 157.868415 61.649) (width 0.5) (layer "F.Cu") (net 10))
 (segment (start 157.46 63) (end 154.92 63) (width 0.5) (layer "F.Cu") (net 8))
 (segment (start 154.92 63) (end 152.12 65.8) (width 0.5) (layer "F.Cu") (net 8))
 (segment (start 161.27 61.6) (end 159.17 59.5) (width 0.5) (layer "F.Cu") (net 6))
 (segment (start 159.17 59.5) (end 152.12 59.5) (width 0.5) (layer "F.Cu") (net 6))
 (segment (start 161.27 63) (end 161.27 61.6) (width 0.5) (layer "F.Cu") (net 6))
 (segment (start 164.5 77) (end 164.5 40.065) (width 0.5) (layer "F.Cu") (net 4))
 (segment (start 162.25 79.25) (end 164.5 77) (width 0.5) (layer "F.Cu") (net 4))
 (segment (start 164.5 40.065) (end 163.305 38.87) (width 0.5) (layer "F.Cu") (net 4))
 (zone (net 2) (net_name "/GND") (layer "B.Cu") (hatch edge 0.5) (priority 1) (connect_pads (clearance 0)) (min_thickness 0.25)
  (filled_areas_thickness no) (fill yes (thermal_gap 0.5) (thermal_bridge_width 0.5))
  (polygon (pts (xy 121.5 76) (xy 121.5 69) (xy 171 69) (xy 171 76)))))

